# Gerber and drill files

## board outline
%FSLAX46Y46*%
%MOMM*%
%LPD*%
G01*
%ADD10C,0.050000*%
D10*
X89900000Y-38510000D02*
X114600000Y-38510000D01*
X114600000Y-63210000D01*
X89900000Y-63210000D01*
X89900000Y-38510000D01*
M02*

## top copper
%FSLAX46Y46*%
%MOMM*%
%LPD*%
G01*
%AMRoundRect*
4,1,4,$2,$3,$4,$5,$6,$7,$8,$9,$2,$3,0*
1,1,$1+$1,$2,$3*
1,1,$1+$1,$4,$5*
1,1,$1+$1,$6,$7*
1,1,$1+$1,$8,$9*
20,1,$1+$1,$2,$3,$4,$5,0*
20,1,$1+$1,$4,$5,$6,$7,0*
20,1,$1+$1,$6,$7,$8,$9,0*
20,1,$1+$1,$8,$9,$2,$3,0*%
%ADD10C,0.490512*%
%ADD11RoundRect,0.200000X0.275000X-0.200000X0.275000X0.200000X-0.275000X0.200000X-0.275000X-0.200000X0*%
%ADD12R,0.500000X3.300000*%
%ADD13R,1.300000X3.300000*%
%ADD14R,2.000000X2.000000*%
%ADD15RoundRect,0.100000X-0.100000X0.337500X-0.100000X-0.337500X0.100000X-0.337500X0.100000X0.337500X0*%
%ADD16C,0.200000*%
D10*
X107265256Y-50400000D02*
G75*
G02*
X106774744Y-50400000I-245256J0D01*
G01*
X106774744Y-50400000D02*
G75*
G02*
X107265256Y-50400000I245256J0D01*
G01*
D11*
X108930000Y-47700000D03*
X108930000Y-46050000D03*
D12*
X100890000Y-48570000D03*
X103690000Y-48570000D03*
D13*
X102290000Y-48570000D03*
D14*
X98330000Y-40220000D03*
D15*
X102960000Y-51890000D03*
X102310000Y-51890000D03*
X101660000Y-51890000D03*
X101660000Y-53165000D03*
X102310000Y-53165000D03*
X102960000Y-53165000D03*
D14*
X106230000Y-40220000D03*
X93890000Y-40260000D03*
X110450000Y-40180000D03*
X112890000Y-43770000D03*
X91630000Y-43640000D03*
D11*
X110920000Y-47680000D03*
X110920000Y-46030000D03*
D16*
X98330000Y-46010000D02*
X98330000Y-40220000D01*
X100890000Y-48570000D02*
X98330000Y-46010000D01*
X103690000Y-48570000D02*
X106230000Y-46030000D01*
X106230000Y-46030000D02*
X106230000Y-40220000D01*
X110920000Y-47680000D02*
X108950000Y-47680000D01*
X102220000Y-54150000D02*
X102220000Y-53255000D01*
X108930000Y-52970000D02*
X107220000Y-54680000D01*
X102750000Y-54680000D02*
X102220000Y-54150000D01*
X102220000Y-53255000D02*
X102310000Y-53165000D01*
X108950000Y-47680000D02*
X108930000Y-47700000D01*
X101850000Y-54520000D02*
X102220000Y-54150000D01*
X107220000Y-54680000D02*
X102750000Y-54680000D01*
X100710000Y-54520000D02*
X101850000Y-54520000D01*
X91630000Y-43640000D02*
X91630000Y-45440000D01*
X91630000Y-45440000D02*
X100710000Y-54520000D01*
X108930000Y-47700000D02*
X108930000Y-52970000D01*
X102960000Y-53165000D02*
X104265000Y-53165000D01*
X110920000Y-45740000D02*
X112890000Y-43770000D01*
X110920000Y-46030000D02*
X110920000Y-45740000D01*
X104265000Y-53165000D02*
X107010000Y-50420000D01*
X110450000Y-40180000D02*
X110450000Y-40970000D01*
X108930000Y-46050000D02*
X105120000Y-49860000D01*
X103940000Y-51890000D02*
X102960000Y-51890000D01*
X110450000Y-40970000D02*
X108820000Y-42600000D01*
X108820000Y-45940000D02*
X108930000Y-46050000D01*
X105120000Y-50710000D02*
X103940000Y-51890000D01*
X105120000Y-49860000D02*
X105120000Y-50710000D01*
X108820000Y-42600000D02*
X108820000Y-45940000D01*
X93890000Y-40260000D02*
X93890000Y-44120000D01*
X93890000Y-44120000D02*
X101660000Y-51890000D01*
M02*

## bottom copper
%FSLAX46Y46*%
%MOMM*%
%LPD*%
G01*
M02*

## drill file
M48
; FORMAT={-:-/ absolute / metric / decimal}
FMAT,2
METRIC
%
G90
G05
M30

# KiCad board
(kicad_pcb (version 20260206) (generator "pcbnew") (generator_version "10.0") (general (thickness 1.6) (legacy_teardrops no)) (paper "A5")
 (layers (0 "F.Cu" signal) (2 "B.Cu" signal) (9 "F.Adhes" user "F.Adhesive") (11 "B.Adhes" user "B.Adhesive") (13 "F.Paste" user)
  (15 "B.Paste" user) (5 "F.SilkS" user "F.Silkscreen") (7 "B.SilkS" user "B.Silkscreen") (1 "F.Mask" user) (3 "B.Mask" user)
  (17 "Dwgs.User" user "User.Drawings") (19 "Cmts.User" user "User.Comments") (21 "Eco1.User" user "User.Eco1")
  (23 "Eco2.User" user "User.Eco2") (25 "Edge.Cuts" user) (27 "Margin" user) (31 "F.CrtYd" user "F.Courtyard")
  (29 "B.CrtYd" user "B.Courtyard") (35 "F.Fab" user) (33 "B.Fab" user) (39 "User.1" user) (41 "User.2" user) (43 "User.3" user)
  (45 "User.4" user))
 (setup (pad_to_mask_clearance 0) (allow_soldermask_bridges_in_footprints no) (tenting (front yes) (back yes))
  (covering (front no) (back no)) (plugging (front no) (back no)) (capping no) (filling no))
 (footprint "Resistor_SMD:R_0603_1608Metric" (layer "F.Cu") (at 108.93 46.875 90)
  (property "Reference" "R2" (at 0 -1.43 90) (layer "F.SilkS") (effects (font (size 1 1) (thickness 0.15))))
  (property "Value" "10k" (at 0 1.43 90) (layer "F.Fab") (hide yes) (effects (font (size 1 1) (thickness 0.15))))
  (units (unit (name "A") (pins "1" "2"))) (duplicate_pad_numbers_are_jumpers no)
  (pad "1" smd roundrect (at -0.825 0 90) (size 0.8 0.95) (layers "F.Cu" "F.Mask" "F.Paste") (roundrect_rratio 0.25) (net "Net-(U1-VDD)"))
  (pad "2" smd roundrect (at 0.825 0 90) (size 0.8 0.95) (layers "F.Cu" "F.Mask" "F.Paste") (roundrect_rratio 0.25) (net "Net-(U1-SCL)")))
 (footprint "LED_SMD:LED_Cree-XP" (layer "F.Cu") (at 102.29 48.57)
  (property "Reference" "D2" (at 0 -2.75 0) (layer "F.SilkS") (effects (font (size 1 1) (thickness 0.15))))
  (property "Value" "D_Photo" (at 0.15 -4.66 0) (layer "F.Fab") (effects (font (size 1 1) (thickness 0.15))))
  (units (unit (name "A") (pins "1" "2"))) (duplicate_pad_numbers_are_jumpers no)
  (pad "" smd rect (at 0 -1) (size 1.01 0.75) (layers "F.Paste"))
  (pad "" smd rect (at 0 0) (size 1.01 0.75) (layers "F.Paste"))
  (pad "" smd rect (at 0 1) (size 1.01 0.75) (layers "F.Paste"))
  (pad "1" smd rect (at -1.4 0) (size 0.5 3.3) (layers "F.Cu" "F.Mask" "F.Paste") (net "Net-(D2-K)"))
  (pad "2" smd rect (at 1.4 0) (size 0.5 3.3) (layers "F.Cu" "F.Mask" "F.Paste") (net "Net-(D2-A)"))
  (pad "3" smd rect (at 0 0) (size 1.3 3.3) (layers "F.Cu" "F.Mask")))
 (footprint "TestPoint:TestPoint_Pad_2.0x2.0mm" (layer "F.Cu") (at 98.33 40.22)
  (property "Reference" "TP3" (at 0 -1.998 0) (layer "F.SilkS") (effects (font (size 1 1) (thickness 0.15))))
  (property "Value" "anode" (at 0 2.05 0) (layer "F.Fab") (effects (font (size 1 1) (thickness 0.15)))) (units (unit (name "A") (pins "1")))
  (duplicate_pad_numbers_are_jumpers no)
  (pad "1" smd rect (at 0 0) (size 2 2) (layers "F.Cu" "F.Mask") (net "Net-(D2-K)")))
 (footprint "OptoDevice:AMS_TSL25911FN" (layer "F.Cu") (at 102.31 52.5275 -90)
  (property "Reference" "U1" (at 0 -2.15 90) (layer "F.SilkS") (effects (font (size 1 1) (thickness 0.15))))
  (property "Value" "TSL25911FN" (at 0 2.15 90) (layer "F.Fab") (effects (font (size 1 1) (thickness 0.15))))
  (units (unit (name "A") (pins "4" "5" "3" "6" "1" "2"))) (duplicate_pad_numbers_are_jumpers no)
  (pad "1" smd roundrect (at -0.6375 -0.65 270) (size 0.875 0.4) (layers "F.Cu" "F.Mask" "F.Paste") (roundrect_rratio 0.25)
   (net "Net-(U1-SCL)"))
  (pad "2" smd roundrect (at -0.6375 0 270) (size 0.875 0.4) (layers "F.Cu" "F.Mask" "F.Paste") (roundrect_rratio 0.25)
   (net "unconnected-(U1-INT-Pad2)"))
  (pad "3" smd roundrect (at -0.6375 0.65 270) (size 0.875 0.4) (layers "F.Cu" "F.Mask" "F.Paste") (roundrect_rratio 0.25)
   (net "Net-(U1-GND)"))
  (pad "4" smd roundrect (at 0.6375 0.65 270) (size 0.875 0.4) (layers "F.Cu" "F.Mask" "F.Paste") (roundrect_rratio 0.25)
   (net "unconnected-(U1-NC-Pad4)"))
  (pad "5" smd roundrect (at 0.6375 0 270) (size 0.875 0.4) (layers "F.Cu" "F.Mask" "F.Paste") (roundrect_rratio 0.25) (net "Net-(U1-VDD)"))
  (pad "6" smd roundrect (at 0.6375 -0.65 270) (size 0.875 0.4) (layers "F.Cu" "F.Mask" "F.Paste") (roundrect_rratio 0.25)
   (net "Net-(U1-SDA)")))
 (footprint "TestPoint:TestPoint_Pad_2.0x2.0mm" (layer "F.Cu") (at 106.23 40.22)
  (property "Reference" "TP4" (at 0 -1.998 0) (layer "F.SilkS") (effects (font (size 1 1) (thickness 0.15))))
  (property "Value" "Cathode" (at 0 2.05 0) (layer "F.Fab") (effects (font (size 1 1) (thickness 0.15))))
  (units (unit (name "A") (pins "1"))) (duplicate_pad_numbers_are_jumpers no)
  (pad "1" smd rect (at 0 0) (size 2 2) (layers "F.Cu" "F.Mask") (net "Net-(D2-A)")))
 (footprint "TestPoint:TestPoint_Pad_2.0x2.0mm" (layer "F.Cu") (at 93.89 40.26)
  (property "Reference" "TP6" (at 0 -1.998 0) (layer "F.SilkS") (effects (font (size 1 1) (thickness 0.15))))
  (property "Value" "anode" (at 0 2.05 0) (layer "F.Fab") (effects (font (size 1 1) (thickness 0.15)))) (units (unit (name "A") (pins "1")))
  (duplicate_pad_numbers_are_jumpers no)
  (pad "1" smd rect (at 0 0) (size 2 2) (layers "F.Cu" "F.Mask") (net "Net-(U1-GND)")))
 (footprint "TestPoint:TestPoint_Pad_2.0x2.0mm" (layer "F.Cu") (at 110.45 40.18)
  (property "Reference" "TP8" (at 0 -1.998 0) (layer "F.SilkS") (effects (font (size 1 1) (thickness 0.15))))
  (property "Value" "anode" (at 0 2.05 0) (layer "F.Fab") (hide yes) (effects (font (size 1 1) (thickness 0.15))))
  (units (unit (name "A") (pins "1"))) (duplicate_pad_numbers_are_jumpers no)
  (pad "1" smd rect (at 0 0) (size 2 2) (layers "F.Cu" "F.Mask") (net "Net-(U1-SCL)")))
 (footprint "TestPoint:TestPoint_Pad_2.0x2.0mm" (layer "F.Cu") (at 112.89 43.77)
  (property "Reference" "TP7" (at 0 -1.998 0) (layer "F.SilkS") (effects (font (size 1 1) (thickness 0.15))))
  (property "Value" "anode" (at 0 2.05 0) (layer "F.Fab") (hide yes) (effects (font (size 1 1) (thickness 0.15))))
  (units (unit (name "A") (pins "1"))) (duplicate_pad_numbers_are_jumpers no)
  (pad "1" smd rect (at 0 0) (size 2 2) (layers "F.Cu" "F.Mask") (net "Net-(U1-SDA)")))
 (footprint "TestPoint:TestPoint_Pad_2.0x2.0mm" (layer "F.Cu") (at 91.63 43.64)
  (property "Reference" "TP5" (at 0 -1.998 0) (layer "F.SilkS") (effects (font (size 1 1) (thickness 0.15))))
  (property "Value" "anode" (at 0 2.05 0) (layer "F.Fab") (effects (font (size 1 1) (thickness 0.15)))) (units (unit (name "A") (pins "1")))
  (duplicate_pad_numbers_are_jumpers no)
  (pad "1" smd rect (at 0 0) (size 2 2) (layers "F.Cu" "F.Mask") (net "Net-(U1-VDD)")))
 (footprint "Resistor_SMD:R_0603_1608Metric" (layer "F.Cu") (at 110.92 46.855 90)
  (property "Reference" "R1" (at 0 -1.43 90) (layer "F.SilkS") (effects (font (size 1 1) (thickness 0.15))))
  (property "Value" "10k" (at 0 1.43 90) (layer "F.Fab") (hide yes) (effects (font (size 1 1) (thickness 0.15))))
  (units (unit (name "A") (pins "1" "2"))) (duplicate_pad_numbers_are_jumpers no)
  (pad "1" smd roundrect (at -0.825 0 90) (size 0.8 0.95) (layers "F.Cu" "F.Mask" "F.Paste") (roundrect_rratio 0.25) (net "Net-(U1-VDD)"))
  (pad "2" smd roundrect (at 0.825 0 90) (size 0.8 0.95) (layers "F.Cu" "F.Mask" "F.Paste") (roundrect_rratio 0.25) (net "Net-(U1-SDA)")))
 (gr_circle (center 107.02 50.4) (end 107.27 50.1) (stroke (width 0.2) (type solid)) (fill yes) (layer "F.Cu") (net "Net-(U1-SDA)"))
 (gr_rect (start 89.9 38.51) (end 114.6 63.21) (stroke (width 0.05) (type solid)) (fill no) (layer "Edge.Cuts"))
 (segment (start 98.33 46.01) (end 98.33 40.22) (width 0.2) (layer "F.Cu") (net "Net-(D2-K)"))
 (segment (start 100.89 48.57) (end 98.33 46.01) (width 0.2) (layer "F.Cu") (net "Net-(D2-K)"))
 (segment (start 103.69 48.57) (end 106.23 46.03) (width 0.2) (layer "F.Cu") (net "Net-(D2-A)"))
 (segment (start 106.23 46.03) (end 106.23 40.22) (width 0.2) (layer "F.Cu") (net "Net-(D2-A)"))
 (segment (start 110.92 47.68) (end 108.95 47.68) (width 0.2) (layer "F.Cu") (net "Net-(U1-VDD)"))
 (segment (start 102.22 54.15) (end 102.22 53.255) (width 0.2) (layer "F.Cu") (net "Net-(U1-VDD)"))
 (segment (start 108.93 52.97) (end 107.22 54.68) (width 0.2) (layer "F.Cu") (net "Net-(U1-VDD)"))
 (segment (start 102.75 54.68) (end 102.22 54.15) (width 0.2) (layer "F.Cu") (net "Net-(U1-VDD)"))
 (segment (start 102.22 53.255) (end 102.31 53.165) (width 0.2) (layer "F.Cu") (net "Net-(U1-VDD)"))
 (segment (start 108.95 47.68) (end 108.93 47.7) (width 0.2) (layer "F.Cu") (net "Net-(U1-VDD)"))
 (segment (start 101.85 54.52) (end 102.22 54.15) (width 0.2) (layer "F.Cu") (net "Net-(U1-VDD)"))
 (segment (start 107.22 54.68) (end 102.75 54.68) (width 0.2) (layer "F.Cu") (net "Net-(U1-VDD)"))
 (segment (start 100.71 54.52) (end 101.85 54.52) (width 0.2) (layer "F.Cu") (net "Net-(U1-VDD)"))
 (segment (start 91.63 43.64) (end 91.63 45.44) (width 0.2) (layer "F.Cu") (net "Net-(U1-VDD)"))
 (segment (start 91.63 45.44) (end 100.71 54.52) (width 0.2) (layer "F.Cu") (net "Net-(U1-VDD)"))
 (segment (start 108.93 47.7) (end 108.93 52.97) (width 0.2) (layer "F.Cu") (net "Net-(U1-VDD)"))
 (segment (start 102.96 53.165) (end 104.265 53.165) (width 0.2) (layer "F.Cu") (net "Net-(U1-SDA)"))
 (segment (start 110.92 45.74) (end 112.89 43.77) (width 0.2) (layer "F.Cu") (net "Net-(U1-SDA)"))
 (segment (start 110.92 46.03) (end 110.92 45.74) (width 0.2) (layer "F.Cu") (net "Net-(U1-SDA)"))
 (segment (start 104.265 53.165) (end 107.01 50.42) (width 0.2) (layer "F.Cu") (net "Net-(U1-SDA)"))
 (segment (start 110.45 40.18) (end 110.45 40.97) (width 0.2) (layer "F.Cu") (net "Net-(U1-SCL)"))
 (segment (start 108.93 46.05) (end 105.12 49.86) (width 0.2) (layer "F.Cu") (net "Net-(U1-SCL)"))
 (segment (start 103.94 51.89) (end 102.96 51.89) (width 0.2) (layer "F.Cu") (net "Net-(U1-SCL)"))
 (segment (start 110.45 40.97) (end 108.82 42.6) (width 0.2) (layer "F.Cu") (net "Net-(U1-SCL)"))
 (segment (start 108.82 45.94) (end 108.93 46.05) (width 0.2) (layer "F.Cu") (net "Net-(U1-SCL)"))
 (segment (start 105.12 50.71) (end 103.94 51.89) (width 0.2) (layer "F.Cu") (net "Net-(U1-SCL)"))
 (segment (start 105.12 49.86) (end 105.12 50.71) (width 0.2) (layer "F.Cu") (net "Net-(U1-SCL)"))
 (segment (start 108.82 42.6) (end 108.82 45.94) (width 0.2) (layer "F.Cu") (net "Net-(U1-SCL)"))
 (segment (start 93.89 40.26) (end 93.89 44.12) (width 0.2) (layer "F.Cu") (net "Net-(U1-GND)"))
 (segment (start 93.89 44.12) (end 101.66 51.89) (width 0.2) (layer "F.Cu") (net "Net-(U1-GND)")))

